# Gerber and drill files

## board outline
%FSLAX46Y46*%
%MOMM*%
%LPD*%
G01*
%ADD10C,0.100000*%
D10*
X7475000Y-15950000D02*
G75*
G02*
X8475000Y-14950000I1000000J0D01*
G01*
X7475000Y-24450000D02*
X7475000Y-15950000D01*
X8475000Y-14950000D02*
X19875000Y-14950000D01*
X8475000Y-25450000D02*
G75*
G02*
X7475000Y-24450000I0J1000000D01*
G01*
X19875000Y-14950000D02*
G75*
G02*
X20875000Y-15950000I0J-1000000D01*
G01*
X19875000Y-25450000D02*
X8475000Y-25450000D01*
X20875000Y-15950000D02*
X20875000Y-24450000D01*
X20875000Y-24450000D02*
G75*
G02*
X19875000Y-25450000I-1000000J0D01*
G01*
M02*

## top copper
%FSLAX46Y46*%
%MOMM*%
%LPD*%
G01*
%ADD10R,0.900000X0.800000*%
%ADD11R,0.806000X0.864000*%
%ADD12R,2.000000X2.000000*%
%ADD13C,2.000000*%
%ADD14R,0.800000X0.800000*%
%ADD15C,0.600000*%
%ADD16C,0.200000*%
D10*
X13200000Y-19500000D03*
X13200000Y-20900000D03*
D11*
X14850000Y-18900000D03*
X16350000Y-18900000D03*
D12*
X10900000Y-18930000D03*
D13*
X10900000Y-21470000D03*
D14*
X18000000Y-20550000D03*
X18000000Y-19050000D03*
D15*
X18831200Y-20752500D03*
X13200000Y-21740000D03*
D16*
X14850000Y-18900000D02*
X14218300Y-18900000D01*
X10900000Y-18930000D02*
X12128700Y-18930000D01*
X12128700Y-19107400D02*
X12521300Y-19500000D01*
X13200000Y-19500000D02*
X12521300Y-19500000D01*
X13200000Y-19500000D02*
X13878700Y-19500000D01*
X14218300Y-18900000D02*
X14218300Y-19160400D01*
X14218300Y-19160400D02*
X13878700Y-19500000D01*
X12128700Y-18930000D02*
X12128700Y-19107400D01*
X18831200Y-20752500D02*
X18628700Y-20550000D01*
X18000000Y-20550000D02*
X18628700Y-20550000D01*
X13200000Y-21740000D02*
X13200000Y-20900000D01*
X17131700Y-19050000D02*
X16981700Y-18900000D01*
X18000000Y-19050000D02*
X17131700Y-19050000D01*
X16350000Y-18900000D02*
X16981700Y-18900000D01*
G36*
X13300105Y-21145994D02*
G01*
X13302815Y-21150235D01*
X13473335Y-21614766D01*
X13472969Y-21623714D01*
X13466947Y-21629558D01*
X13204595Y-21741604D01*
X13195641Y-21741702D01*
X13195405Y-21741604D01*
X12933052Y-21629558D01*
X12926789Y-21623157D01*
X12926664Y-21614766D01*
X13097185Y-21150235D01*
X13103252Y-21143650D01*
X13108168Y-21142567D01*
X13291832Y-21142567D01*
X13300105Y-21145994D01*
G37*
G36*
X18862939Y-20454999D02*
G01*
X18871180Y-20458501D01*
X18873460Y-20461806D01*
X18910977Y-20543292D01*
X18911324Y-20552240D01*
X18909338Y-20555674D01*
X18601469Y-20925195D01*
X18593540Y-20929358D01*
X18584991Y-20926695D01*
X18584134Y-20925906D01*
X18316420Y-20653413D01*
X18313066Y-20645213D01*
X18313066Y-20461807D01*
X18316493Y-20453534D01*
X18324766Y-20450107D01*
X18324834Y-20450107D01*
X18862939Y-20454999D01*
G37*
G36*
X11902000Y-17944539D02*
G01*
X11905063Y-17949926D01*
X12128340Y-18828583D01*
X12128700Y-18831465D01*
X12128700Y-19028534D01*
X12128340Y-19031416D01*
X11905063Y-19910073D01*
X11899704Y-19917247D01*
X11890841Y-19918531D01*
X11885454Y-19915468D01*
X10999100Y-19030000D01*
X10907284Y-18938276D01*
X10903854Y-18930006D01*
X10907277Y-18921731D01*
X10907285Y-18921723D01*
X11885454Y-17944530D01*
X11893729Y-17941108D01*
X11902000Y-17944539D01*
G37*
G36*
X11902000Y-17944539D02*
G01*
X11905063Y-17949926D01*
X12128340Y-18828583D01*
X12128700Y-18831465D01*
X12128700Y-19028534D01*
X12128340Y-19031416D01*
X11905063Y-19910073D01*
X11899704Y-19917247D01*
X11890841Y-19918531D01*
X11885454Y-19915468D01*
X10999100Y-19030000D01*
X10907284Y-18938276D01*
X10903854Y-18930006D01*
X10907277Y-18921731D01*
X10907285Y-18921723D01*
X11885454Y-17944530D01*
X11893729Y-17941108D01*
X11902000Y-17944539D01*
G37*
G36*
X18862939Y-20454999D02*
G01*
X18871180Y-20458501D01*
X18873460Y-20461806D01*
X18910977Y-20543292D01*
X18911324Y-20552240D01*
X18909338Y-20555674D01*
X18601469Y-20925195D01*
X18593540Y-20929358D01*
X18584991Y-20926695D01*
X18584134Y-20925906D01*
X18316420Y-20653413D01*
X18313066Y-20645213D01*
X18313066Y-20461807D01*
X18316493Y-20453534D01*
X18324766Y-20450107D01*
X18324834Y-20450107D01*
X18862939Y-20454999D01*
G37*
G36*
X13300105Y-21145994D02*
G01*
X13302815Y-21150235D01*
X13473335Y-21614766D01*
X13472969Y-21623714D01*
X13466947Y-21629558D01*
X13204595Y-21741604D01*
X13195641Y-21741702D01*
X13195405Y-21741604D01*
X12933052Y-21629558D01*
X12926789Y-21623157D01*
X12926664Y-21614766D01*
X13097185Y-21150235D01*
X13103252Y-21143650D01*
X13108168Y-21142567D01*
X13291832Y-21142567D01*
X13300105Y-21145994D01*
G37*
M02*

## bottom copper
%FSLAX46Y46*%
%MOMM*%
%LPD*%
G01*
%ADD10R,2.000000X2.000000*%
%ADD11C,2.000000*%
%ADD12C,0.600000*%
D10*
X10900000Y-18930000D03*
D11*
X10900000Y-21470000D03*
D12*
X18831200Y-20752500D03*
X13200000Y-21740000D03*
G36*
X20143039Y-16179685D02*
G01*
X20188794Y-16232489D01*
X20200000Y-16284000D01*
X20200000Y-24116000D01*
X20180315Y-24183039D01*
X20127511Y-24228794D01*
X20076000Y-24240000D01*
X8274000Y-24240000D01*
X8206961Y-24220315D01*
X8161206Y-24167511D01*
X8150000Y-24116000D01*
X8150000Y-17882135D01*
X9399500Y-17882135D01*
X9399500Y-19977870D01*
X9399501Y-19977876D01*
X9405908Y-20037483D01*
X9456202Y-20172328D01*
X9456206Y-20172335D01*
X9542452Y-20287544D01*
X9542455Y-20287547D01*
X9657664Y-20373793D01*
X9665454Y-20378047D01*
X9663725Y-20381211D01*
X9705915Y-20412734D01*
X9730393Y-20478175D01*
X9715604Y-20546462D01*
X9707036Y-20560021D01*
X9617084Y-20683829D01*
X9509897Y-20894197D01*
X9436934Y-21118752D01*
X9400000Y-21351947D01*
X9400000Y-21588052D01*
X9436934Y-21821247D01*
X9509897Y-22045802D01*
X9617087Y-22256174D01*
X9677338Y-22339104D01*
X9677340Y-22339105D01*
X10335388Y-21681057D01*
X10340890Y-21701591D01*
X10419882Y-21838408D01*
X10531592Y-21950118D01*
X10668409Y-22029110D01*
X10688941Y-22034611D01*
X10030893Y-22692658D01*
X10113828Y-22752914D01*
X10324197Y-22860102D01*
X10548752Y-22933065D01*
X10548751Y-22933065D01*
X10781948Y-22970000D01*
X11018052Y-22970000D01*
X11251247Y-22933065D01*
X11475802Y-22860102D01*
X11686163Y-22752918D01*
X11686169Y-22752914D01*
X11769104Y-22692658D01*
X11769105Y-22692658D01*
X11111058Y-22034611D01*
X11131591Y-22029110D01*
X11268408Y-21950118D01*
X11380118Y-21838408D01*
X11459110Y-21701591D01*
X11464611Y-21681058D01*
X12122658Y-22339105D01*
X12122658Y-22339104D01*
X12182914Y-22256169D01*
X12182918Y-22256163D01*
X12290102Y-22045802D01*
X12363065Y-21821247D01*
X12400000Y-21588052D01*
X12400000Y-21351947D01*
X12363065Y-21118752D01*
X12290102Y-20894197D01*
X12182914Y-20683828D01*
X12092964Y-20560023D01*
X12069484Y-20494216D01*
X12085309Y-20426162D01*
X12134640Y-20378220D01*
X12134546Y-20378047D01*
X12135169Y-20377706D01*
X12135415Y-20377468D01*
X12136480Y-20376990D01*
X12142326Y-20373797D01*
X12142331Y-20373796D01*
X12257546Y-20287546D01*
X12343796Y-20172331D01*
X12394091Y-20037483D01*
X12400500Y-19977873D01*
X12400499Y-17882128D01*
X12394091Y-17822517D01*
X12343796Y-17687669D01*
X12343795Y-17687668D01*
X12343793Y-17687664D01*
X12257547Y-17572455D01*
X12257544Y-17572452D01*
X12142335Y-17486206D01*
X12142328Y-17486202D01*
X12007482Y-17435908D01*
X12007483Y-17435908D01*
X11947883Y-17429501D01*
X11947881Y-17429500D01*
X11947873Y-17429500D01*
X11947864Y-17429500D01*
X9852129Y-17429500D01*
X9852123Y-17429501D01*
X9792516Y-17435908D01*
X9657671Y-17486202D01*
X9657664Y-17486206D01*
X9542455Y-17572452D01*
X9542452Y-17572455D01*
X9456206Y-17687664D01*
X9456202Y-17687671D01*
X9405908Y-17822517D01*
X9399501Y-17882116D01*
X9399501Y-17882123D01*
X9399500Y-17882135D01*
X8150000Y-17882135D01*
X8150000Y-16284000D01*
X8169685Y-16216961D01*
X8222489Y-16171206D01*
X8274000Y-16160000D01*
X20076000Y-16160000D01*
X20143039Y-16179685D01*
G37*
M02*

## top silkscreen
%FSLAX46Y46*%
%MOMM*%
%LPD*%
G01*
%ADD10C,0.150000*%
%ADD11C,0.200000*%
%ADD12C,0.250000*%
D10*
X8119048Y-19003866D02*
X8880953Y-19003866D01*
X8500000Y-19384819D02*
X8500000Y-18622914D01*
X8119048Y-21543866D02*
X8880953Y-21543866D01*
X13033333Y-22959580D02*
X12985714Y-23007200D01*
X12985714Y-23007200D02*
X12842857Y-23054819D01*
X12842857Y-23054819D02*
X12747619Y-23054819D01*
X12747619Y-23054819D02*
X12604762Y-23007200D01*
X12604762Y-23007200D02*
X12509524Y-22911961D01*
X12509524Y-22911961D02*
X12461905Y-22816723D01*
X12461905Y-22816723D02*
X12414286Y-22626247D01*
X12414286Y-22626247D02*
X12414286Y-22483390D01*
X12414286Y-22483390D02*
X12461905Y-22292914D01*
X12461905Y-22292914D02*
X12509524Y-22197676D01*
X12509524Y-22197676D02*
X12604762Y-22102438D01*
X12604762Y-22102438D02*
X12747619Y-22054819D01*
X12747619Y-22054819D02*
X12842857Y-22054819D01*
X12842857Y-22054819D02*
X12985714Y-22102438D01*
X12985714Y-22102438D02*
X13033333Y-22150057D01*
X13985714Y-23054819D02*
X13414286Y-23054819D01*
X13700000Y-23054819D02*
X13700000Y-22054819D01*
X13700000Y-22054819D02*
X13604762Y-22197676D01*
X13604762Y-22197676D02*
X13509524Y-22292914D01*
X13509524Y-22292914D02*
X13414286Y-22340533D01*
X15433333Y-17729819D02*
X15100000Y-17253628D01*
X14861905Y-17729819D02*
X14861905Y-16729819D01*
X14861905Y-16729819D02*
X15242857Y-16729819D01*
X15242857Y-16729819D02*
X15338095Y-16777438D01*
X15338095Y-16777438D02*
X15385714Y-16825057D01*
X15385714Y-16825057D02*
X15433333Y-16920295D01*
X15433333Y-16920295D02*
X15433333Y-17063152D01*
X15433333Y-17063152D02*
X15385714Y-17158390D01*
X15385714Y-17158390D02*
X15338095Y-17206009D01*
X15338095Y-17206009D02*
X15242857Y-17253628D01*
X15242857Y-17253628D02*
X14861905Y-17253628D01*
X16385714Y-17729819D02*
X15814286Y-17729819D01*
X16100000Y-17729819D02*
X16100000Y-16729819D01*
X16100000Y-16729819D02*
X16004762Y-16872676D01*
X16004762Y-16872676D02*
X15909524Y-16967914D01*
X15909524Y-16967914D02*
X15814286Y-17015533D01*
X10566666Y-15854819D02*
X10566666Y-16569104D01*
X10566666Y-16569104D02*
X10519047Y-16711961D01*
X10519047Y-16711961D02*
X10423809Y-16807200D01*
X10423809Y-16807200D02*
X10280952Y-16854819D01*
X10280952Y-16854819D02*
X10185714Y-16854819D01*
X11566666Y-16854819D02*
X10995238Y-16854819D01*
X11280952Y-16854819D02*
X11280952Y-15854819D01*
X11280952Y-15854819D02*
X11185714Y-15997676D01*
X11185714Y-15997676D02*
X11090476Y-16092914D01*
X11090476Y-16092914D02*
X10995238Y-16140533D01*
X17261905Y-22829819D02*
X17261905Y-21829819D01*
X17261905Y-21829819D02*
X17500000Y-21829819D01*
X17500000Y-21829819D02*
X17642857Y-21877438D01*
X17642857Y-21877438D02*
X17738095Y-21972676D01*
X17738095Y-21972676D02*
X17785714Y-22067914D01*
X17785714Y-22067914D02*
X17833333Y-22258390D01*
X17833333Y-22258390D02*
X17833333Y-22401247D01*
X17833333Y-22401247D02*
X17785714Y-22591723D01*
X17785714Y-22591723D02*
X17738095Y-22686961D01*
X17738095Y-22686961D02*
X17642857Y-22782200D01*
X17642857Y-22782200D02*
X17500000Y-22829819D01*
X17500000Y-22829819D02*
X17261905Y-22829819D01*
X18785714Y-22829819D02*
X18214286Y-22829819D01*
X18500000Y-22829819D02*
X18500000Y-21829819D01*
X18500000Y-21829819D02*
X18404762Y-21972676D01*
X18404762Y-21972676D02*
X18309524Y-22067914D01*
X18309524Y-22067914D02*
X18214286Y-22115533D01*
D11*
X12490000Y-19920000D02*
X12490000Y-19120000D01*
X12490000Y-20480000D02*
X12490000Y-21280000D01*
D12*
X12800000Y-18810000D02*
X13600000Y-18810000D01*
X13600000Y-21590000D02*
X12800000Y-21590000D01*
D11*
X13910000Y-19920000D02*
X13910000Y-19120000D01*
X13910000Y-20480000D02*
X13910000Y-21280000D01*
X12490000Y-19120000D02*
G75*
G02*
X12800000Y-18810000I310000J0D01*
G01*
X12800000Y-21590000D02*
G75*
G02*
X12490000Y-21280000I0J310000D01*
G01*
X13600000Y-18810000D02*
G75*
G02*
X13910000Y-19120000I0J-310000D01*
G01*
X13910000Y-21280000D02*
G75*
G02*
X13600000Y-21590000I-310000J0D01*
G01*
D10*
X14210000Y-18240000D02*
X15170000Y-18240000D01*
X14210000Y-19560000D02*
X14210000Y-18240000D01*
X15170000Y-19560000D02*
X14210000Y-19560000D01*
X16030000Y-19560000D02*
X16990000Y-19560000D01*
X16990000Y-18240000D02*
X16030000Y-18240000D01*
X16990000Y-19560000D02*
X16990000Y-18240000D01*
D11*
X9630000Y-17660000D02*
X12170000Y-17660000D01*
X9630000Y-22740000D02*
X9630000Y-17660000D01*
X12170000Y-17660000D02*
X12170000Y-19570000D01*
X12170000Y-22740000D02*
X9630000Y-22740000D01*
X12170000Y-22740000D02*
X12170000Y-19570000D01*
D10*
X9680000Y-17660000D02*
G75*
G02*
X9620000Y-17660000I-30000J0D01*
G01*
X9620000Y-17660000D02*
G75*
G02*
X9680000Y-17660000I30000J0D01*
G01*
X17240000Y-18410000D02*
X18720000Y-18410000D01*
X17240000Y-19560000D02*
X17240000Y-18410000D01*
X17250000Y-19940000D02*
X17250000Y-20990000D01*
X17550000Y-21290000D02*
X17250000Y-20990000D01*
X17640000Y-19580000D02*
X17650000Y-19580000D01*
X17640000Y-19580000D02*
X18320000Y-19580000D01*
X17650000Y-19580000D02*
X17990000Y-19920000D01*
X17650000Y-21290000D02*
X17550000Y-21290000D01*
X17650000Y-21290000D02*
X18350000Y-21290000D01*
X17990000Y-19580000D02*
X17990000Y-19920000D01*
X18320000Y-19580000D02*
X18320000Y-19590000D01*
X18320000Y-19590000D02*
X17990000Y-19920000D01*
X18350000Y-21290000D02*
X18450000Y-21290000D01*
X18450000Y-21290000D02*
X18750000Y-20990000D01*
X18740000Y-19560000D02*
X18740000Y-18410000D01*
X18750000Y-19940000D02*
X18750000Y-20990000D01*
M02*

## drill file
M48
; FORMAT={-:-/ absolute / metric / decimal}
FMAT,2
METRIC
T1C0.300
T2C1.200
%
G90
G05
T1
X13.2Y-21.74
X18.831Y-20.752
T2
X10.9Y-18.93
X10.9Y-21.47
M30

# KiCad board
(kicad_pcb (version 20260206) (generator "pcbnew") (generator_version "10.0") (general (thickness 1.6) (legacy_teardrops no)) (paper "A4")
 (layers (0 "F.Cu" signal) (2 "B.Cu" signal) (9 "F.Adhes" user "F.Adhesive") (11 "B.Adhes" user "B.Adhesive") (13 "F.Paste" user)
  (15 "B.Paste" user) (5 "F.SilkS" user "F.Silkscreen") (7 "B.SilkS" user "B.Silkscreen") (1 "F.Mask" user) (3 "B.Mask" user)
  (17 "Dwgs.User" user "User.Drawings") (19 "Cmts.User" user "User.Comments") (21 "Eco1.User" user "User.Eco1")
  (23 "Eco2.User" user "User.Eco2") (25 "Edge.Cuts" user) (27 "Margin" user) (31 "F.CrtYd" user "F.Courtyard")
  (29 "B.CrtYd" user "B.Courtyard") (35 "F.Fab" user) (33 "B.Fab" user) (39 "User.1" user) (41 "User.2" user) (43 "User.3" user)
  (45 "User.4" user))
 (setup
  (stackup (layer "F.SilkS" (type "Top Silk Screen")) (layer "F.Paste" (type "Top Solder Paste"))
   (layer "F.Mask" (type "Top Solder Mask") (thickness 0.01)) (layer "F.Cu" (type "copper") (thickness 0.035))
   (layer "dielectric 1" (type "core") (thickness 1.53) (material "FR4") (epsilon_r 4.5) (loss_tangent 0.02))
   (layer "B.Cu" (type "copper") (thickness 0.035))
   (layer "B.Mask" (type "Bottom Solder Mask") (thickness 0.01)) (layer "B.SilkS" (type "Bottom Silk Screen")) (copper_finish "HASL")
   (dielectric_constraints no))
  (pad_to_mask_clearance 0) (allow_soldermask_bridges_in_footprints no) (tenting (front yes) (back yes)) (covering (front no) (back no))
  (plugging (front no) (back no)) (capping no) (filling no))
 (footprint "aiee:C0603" (layer "F.Cu") (at 13.2 20.2 -90)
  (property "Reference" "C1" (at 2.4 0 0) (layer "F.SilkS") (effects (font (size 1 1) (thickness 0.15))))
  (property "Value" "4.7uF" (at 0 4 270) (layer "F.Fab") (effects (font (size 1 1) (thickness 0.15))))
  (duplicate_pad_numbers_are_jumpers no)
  (fp_line (start -0.28 0.71) (end -1.08 0.71) (stroke (width 0.2) (type solid)) (layer "F.SilkS"))
  (fp_line (start 0.28 0.71) (end 1.08 0.71) (stroke (width 0.2) (type solid)) (layer "F.SilkS"))
  (fp_line (start -1.39 0.4) (end -1.39 -0.4) (stroke (width 0.25) (type solid)) (layer "F.SilkS"))
  (fp_line (start 1.39 -0.4) (end 1.39 0.4) (stroke (width 0.25) (type solid)) (layer "F.SilkS"))
  (fp_line (start -0.28 -0.71) (end -1.08 -0.71) (stroke (width 0.2) (type solid)) (layer "F.SilkS"))
  (fp_line (start 0.28 -0.71) (end 1.08 -0.71) (stroke (width 0.2) (type solid)) (layer "F.SilkS"))
  (fp_arc (start -1.08 0.71) (mid -1.299203 0.619203) (end -1.39 0.4) (stroke (width 0.2) (type solid)) (layer "F.SilkS"))
  (fp_arc (start 1.39 0.4) (mid 1.299203 0.619203) (end 1.08 0.71) (stroke (width 0.2) (type solid)) (layer "F.SilkS"))
  (fp_arc (start -1.39 -0.4) (mid -1.299203 -0.619203) (end -1.08 -0.71) (stroke (width 0.2) (type solid)) (layer "F.SilkS"))
  (fp_arc (start 1.08 -0.71) (mid 1.299203 -0.619203) (end 1.39 -0.4) (stroke (width 0.2) (type solid)) (layer "F.SilkS"))
  (pad "1" smd rect (at -0.7 0 270) (size 0.8 0.9) (layers "F.Cu" "F.Mask" "F.Paste") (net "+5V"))
  (pad "2" smd rect (at 0.7 0 270) (size 0.8 0.9) (layers "F.Cu" "F.Mask" "F.Paste") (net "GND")))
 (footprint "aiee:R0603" (layer "F.Cu") (at 15.6 18.9)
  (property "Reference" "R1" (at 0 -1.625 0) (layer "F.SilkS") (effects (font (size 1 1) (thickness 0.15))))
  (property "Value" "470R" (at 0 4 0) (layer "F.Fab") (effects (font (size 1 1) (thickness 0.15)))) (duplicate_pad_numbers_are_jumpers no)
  (fp_line (start -1.39 -0.66) (end -0.43 -0.66) (stroke (width 0.15) (type solid)) (layer "F.SilkS"))
  (fp_line (start -1.39 0.66) (end -1.39 -0.66) (stroke (width 0.15) (type solid)) (layer "F.SilkS"))
  (fp_line (start -0.43 0.66) (end -1.39 0.66) (stroke (width 0.15) (type solid)) (layer "F.SilkS"))
  (fp_line (start 0.43 0.66) (end 1.39 0.66) (stroke (width 0.15) (type solid)) (layer "F.SilkS"))
  (fp_line (start 1.39 -0.66) (end 0.43 -0.66) (stroke (width 0.15) (type solid)) (layer "F.SilkS"))
  (fp_line (start 1.39 0.66) (end 1.39 -0.66) (stroke (width 0.15) (type solid)) (layer "F.SilkS"))
  (pad "1" smd rect (at -0.75 0) (size 0.806 0.864) (layers "F.Cu" "F.Mask" "F.Paste") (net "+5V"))
  (pad "2" smd rect (at 0.75 0) (size 0.806 0.864) (layers "F.Cu" "F.Mask" "F.Paste") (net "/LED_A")))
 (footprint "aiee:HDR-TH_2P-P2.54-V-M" (layer "F.Cu") (at 10.9 20.2 -90)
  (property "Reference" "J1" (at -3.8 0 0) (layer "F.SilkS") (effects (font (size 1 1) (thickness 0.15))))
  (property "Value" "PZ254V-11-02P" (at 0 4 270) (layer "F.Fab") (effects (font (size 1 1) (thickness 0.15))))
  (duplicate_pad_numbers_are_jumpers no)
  (fp_line (start -2.54 1.27) (end -2.54 -1.27) (stroke (width 0.2) (type solid)) (layer "F.SilkS"))
  (fp_line (start 2.54 1.27) (end -2.54 1.27) (stroke (width 0.2) (type solid)) (layer "F.SilkS"))
  (fp_line (start -2.54 -1.27) (end -0.63 -1.27) (stroke (width 0.2) (type solid)) (layer "F.SilkS"))
  (fp_line (start 2.54 -1.27) (end 2.54 1.27) (stroke (width 0.2) (type solid)) (layer "F.SilkS"))
  (fp_line (start 2.54 -1.27) (end -0.63 -1.27) (stroke (width 0.2) (type solid)) (layer "F.SilkS"))
  (fp_circle (center -2.54 1.25) (end -2.51 1.25) (stroke (width 0.15) (type solid)) (fill no) (layer "F.SilkS"))
  (pad "1" thru_hole rect (at -1.27 0 270) (size 2 2) (drill 1.199998) (layers "*.Cu" "*.Mask") (remove_unused_layers no) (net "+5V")
   (teardrops (best_length_ratio 0.5) (max_length 1) (best_width_ratio 1) (max_width 2) (curved_edges no) (filter_ratio 0.9) (enabled yes)
    (allow_two_segments yes) (prefer_zone_connections yes)))
  (pad "2" thru_hole circle (at 1.27 0 270) (size 2 2) (drill 1.199998) (layers "*.Cu" "*.Mask") (remove_unused_layers no) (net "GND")))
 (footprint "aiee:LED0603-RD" (layer "F.Cu") (at 18 19.8 90)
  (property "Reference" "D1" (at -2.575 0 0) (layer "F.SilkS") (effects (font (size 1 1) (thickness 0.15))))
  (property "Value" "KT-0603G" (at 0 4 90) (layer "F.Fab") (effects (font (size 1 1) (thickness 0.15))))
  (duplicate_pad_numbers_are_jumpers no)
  (fp_line (start 1.39 -0.76) (end 1.39 0.72) (stroke (width 0.15) (type solid)) (layer "F.SilkS"))
  (fp_line (start 0.24 -0.76) (end 1.39 -0.76) (stroke (width 0.15) (type solid)) (layer "F.SilkS"))
  (fp_line (start -0.14 -0.75) (end -1.19 -0.75) (stroke (width 0.15) (type solid)) (layer "F.SilkS"))
  (fp_line (start -1.49 -0.45) (end -1.19 -0.75) (stroke (width 0.15) (type solid)) (layer "F.SilkS"))
  (fp_line (start 0.22 -0.36) (end 0.22 -0.35) (stroke (width 0.15) (type solid)) (layer "F.SilkS"))
  (fp_line (start 0.22 -0.36) (end 0.22 0.32) (stroke (width 0.15) (type solid)) (layer "F.SilkS"))
  (fp_line (start 0.22 -0.35) (end -0.12 -0.01) (stroke (width 0.15) (type solid)) (layer "F.SilkS"))
  (fp_line (start -1.49 -0.35) (end -1.49 -0.45) (stroke (width 0.15) (type solid)) (layer "F.SilkS"))
  (fp_line (start -1.49 -0.35) (end -1.49 0.35) (stroke (width 0.15) (type solid)) (layer "F.SilkS"))
  (fp_line (start 0.22 -0.01) (end -0.12 -0.01) (stroke (width 0.15) (type solid)) (layer "F.SilkS"))
  (fp_line (start 0.22 0.32) (end 0.21 0.32) (stroke (width 0.15) (type solid)) (layer "F.SilkS"))
  (fp_line (start 0.21 0.32) (end -0.12 -0.01) (stroke (width 0.15) (type solid)) (layer "F.SilkS"))
  (fp_line (start -1.49 0.35) (end -1.49 0.45) (stroke (width 0.15) (type solid)) (layer "F.SilkS"))
  (fp_line (start -1.49 0.45) (end -1.19 0.75) (stroke (width 0.15) (type solid)) (layer "F.SilkS"))
  (fp_line (start 0.24 0.74) (end 1.39 0.74) (stroke (width 0.15) (type solid)) (layer "F.SilkS"))
  (fp_line (start -0.14 0.75) (end -1.19 0.75) (stroke (width 0.15) (type solid)) (layer "F.SilkS"))
  (pad "1" smd rect (at -0.75 0 180) (size 0.8 0.8) (layers "F.Cu" "F.Mask" "F.Paste") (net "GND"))
  (pad "2" smd rect (at 0.75 0 180) (size 0.8 0.8) (layers "F.Cu" "F.Mask" "F.Paste") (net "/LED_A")))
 (gr_arc (start 7.475 15.95) (mid 7.767893 15.242893) (end 8.475 14.95) (stroke (width 0.1) (type default)) (layer "Edge.Cuts"))
 (gr_line (start 7.475 24.45) (end 7.475 15.95) (stroke (width 0.1) (type default)) (layer "Edge.Cuts"))
 (gr_line (start 8.475 14.95) (end 19.875 14.95) (stroke (width 0.1) (type default)) (layer "Edge.Cuts"))
 (gr_arc (start 8.475 25.45) (mid 7.767893 25.157106) (end 7.475 24.45) (stroke (width 0.1) (type default)) (layer "Edge.Cuts"))
 (gr_arc (start 19.875 14.95) (mid 20.582106 15.242893) (end 20.875 15.95) (stroke (width 0.1) (type default)) (layer "Edge.Cuts"))
 (gr_line (start 19.875 25.45) (end 8.475 25.45) (stroke (width 0.1) (type default)) (layer "Edge.Cuts"))
 (gr_line (start 20.875 15.95) (end 20.875 24.45) (stroke (width 0.1) (type default)) (layer "Edge.Cuts"))
 (gr_arc (start 20.875 24.45) (mid 20.582106 25.157106) (end 19.875 25.45) (stroke (width 0.1) (type default)) (layer "Edge.Cuts"))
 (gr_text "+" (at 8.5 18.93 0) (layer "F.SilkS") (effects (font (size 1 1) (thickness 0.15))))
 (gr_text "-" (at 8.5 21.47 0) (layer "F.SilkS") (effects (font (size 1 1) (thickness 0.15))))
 (segment (start 14.85 18.9) (end 14.2183 18.9) (width 0.2) (layer "F.Cu") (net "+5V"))
 (segment (start 10.9 18.93) (end 12.1287 18.93) (width 0.2) (layer "F.Cu") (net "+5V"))
 (segment (start 12.1287 19.1074) (end 12.5213 19.5) (width 0.2) (layer "F.Cu") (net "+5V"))
 (segment (start 13.2 19.5) (end 12.5213 19.5) (width 0.2) (layer "F.Cu") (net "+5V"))
 (segment (start 13.2 19.5) (end 13.8787 19.5) (width 0.2) (layer "F.Cu") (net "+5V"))
 (segment (start 14.2183 18.9) (end 14.2183 19.1604) (width 0.2) (layer "F.Cu") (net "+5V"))
 (segment (start 14.2183 19.1604) (end 13.8787 19.5) (width 0.2) (layer "F.Cu") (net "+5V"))
 (segment (start 12.1287 18.93) (end 12.1287 19.1074) (width 0.2) (layer "F.Cu") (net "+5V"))
 (segment (start 18.8312 20.7525) (end 18.6287 20.55) (width 0.2) (layer "F.Cu") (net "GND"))
 (segment (start 18 20.55) (end 18.6287 20.55) (width 0.2) (layer "F.Cu") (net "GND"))
 (segment (start 13.2 21.74) (end 13.2 20.9) (width 0.2) (layer "F.Cu") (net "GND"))
 (via (at 18.8312 20.7525) (size 0.6) (drill 0.3) (layers "F.Cu" "B.Cu")
  (teardrops (best_length_ratio 0.5) (max_length 1) (best_width_ratio 1) (max_width 2) (curved_edges no) (filter_ratio 0.9) (enabled yes)
   (allow_two_segments yes) (prefer_zone_connections yes))
  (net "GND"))
 (via (at 13.2 21.74) (size 0.6) (drill 0.3) (layers "F.Cu" "B.Cu")
  (teardrops (best_length_ratio 0.5) (max_length 1) (best_width_ratio 1) (max_width 2) (curved_edges no) (filter_ratio 0.9) (enabled yes)
   (allow_two_segments yes) (prefer_zone_connections yes))
  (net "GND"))
 (segment (start 17.1317 19.05) (end 16.9817 18.9) (width 0.2) (layer "F.Cu") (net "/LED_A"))
 (segment (start 18 19.05) (end 17.1317 19.05) (width 0.2) (layer "F.Cu") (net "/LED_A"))
 (segment (start 16.35 18.9) (end 16.9817 18.9) (width 0.2) (layer "F.Cu") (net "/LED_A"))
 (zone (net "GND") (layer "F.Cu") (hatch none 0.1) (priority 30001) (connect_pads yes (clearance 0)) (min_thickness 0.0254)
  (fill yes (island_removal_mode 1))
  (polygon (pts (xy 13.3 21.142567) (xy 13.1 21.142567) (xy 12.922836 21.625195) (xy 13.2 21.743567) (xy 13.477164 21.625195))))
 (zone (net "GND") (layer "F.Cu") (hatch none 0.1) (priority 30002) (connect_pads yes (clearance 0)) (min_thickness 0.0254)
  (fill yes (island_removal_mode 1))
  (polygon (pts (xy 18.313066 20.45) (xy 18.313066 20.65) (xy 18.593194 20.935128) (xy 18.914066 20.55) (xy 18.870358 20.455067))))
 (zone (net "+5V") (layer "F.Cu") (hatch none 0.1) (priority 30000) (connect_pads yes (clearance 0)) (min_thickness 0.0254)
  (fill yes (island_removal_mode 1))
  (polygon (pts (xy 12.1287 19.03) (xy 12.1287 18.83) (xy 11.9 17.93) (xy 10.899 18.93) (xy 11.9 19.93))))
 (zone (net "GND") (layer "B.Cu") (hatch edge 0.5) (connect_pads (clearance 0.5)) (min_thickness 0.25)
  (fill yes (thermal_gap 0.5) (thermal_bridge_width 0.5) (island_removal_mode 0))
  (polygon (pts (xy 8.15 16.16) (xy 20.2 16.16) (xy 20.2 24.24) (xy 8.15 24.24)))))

